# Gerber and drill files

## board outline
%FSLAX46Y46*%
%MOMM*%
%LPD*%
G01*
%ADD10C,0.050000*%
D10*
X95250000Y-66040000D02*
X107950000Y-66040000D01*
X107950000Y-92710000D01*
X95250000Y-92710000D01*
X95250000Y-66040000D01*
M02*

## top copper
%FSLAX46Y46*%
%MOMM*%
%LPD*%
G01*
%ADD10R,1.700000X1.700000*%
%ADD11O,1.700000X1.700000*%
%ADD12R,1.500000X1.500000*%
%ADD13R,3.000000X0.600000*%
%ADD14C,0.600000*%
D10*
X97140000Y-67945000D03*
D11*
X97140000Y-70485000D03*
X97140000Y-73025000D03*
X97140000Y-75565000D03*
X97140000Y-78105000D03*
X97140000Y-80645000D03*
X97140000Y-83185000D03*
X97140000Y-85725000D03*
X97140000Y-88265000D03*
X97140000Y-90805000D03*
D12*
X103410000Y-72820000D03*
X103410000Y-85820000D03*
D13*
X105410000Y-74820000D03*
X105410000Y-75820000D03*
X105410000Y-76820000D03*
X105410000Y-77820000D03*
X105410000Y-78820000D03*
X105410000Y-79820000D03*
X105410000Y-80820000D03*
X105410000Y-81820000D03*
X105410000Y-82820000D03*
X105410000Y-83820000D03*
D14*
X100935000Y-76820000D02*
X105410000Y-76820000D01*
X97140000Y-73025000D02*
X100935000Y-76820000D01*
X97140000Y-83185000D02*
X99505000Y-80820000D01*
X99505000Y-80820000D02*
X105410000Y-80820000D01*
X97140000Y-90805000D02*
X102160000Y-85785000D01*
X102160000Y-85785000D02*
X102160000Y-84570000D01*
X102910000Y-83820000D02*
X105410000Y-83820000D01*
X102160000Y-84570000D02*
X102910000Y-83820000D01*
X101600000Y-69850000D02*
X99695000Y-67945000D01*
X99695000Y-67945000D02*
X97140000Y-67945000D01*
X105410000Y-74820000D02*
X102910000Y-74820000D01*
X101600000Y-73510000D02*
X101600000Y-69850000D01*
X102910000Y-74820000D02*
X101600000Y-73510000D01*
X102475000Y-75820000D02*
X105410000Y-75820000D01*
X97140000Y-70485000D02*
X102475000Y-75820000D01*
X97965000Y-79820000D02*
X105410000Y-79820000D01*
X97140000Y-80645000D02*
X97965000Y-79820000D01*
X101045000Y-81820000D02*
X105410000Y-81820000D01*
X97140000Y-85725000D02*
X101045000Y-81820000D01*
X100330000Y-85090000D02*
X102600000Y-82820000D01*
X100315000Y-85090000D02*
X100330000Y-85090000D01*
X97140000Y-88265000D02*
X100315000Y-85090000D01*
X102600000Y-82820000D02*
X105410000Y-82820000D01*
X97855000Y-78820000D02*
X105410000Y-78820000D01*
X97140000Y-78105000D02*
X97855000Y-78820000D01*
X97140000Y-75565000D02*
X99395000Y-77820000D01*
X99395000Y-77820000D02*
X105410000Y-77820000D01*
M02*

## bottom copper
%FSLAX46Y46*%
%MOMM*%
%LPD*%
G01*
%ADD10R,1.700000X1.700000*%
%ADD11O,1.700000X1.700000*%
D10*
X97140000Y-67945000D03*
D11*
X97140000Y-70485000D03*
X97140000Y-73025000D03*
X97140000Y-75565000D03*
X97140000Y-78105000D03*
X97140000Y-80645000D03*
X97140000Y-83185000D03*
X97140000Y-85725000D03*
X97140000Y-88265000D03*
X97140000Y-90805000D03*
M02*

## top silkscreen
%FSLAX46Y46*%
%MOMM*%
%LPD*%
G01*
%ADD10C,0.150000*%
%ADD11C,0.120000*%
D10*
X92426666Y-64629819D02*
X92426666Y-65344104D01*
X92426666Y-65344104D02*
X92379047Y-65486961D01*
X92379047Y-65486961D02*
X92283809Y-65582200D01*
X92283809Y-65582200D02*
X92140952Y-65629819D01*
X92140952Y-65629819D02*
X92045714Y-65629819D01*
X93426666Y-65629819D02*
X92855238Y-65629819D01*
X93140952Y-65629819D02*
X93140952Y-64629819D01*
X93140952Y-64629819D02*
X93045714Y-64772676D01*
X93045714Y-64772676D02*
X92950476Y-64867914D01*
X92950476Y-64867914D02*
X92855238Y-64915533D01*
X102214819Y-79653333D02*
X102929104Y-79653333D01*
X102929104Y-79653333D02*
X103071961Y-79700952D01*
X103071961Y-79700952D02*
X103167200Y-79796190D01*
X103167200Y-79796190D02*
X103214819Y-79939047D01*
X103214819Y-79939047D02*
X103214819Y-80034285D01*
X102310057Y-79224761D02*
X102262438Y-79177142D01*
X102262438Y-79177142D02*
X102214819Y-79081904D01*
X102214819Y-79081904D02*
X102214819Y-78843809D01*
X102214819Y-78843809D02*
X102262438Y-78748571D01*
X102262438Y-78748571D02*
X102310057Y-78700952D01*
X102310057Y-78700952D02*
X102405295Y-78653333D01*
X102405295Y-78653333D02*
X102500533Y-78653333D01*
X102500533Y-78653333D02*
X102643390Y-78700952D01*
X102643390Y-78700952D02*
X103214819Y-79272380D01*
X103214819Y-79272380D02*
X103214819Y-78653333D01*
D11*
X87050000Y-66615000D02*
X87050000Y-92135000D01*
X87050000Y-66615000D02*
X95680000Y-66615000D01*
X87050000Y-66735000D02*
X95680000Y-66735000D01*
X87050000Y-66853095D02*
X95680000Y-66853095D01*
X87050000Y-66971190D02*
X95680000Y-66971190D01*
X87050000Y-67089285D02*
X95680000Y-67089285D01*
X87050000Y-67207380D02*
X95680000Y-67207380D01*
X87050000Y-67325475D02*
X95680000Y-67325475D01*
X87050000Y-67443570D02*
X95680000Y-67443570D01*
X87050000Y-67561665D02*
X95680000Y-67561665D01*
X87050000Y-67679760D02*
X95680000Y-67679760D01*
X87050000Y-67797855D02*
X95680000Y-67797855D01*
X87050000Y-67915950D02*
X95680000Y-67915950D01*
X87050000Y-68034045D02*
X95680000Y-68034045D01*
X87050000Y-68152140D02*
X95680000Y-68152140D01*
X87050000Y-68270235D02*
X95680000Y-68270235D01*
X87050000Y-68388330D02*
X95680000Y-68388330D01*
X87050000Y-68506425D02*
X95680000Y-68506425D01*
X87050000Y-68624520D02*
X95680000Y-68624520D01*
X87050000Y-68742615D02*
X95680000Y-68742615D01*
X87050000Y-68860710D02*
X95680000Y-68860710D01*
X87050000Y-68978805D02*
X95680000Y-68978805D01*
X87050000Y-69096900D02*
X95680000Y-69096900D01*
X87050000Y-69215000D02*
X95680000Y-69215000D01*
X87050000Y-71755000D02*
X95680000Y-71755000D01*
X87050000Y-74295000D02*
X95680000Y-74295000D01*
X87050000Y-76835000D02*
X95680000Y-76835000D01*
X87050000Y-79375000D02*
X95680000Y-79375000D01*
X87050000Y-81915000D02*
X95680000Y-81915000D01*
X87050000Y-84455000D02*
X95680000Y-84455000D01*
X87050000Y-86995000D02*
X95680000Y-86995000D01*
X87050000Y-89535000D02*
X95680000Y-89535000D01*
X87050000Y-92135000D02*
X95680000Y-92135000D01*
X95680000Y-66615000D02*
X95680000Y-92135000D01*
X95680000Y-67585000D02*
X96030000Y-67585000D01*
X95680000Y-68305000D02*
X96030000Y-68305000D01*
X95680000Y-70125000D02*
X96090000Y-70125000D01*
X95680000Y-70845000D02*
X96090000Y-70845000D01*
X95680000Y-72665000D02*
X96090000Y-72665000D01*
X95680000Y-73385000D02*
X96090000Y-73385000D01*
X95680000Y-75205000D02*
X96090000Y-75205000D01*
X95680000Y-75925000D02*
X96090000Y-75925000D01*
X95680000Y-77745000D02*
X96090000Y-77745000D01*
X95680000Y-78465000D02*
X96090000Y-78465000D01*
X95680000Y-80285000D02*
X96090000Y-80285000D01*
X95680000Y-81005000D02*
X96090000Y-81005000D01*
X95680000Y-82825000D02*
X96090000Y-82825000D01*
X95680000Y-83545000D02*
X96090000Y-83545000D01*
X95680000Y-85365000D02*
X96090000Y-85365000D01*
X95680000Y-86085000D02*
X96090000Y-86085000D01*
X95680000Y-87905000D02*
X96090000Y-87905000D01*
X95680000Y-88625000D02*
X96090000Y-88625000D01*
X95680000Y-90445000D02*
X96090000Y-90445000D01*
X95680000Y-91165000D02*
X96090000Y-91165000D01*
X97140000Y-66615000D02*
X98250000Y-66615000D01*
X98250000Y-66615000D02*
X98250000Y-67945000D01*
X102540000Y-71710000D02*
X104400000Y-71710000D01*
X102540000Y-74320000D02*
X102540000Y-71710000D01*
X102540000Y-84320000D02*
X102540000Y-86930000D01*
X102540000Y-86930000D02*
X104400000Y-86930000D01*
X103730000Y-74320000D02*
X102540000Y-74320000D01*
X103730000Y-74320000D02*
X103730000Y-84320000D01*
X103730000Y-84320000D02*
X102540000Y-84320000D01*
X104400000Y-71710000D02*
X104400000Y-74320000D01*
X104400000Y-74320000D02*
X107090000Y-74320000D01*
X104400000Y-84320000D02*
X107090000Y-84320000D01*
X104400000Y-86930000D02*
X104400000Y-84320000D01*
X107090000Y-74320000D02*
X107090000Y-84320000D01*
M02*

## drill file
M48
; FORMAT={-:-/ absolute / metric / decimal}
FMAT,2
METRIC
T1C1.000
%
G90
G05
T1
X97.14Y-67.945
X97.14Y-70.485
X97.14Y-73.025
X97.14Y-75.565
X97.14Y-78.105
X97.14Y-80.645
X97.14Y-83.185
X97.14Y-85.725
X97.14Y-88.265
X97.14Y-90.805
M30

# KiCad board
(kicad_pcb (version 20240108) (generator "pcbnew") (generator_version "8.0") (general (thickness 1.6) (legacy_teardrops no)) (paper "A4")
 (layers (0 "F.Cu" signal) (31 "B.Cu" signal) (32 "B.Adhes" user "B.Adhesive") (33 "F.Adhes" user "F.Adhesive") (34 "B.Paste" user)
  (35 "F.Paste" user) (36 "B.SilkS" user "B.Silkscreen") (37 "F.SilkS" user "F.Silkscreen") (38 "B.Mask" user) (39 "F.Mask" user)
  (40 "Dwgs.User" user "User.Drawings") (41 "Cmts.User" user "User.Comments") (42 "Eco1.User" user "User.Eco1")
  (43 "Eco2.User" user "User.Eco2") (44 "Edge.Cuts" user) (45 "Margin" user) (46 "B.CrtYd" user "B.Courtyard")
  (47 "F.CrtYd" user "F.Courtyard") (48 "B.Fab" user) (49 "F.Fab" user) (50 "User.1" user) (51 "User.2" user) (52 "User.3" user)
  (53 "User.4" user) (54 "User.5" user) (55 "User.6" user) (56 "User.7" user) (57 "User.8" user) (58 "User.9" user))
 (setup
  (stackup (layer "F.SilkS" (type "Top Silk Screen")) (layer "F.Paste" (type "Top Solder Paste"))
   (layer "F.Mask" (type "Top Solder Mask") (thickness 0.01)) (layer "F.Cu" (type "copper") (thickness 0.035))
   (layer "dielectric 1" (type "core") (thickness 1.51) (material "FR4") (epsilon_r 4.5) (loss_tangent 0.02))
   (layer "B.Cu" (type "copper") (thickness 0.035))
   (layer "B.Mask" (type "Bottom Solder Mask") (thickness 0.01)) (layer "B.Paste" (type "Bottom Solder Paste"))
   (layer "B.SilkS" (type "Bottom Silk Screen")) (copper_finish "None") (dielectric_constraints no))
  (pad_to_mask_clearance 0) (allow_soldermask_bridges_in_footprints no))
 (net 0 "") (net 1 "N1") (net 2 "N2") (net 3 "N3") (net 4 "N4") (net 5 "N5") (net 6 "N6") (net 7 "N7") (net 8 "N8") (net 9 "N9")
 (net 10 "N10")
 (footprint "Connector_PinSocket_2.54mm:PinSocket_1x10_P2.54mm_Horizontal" (layer "F.Cu") (at 97.14 67.945)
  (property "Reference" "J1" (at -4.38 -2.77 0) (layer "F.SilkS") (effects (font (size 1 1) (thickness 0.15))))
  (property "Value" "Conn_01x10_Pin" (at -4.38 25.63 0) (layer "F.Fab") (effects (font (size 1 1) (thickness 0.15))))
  (fp_line (start -10.09 -1.33) (end -10.09 24.19) (stroke (width 0.12) (type solid)) (layer "F.SilkS"))
  (fp_line (start -10.09 -1.33) (end -1.46 -1.33) (stroke (width 0.12) (type solid)) (layer "F.SilkS"))
  (fp_line (start -10.09 -1.21) (end -1.46 -1.21) (stroke (width 0.12) (type solid)) (layer "F.SilkS"))
  (fp_line (start -10.09 -1.091905) (end -1.46 -1.091905) (stroke (width 0.12) (type solid)) (layer "F.SilkS"))
  (fp_line (start -10.09 -0.97381) (end -1.46 -0.97381) (stroke (width 0.12) (type solid)) (layer "F.SilkS"))
  (fp_line (start -10.09 -0.855715) (end -1.46 -0.855715) (stroke (width 0.12) (type solid)) (layer "F.SilkS"))
  (fp_line (start -10.09 -0.73762) (end -1.46 -0.73762) (stroke (width 0.12) (type solid)) (layer "F.SilkS"))
  (fp_line (start -10.09 -0.619525) (end -1.46 -0.619525) (stroke (width 0.12) (type solid)) (layer "F.SilkS"))
  (fp_line (start -10.09 -0.50143) (end -1.46 -0.50143) (stroke (width 0.12) (type solid)) (layer "F.SilkS"))
  (fp_line (start -10.09 -0.383335) (end -1.46 -0.383335) (stroke (width 0.12) (type solid)) (layer "F.SilkS"))
  (fp_line (start -10.09 -0.26524) (end -1.46 -0.26524) (stroke (width 0.12) (type solid)) (layer "F.SilkS"))
  (fp_line (start -10.09 -0.147145) (end -1.46 -0.147145) (stroke (width 0.12) (type solid)) (layer "F.SilkS"))
  (fp_line (start -10.09 -0.02905) (end -1.46 -0.02905) (stroke (width 0.12) (type solid)) (layer "F.SilkS"))
  (fp_line (start -10.09 0.089045) (end -1.46 0.089045) (stroke (width 0.12) (type solid)) (layer "F.SilkS"))
  (fp_line (start -10.09 0.20714) (end -1.46 0.20714) (stroke (width 0.12) (type solid)) (layer "F.SilkS"))
  (fp_line (start -10.09 0.325235) (end -1.46 0.325235) (stroke (width 0.12) (type solid)) (layer "F.SilkS"))
  (fp_line (start -10.09 0.44333) (end -1.46 0.44333) (stroke (width 0.12) (type solid)) (layer "F.SilkS"))
  (fp_line (start -10.09 0.561425) (end -1.46 0.561425) (stroke (width 0.12) (type solid)) (layer "F.SilkS"))
  (fp_line (start -10.09 0.67952) (end -1.46 0.67952) (stroke (width 0.12) (type solid)) (layer "F.SilkS"))
  (fp_line (start -10.09 0.797615) (end -1.46 0.797615) (stroke (width 0.12) (type solid)) (layer "F.SilkS"))
  (fp_line (start -10.09 0.91571) (end -1.46 0.91571) (stroke (width 0.12) (type solid)) (layer "F.SilkS"))
  (fp_line (start -10.09 1.033805) (end -1.46 1.033805) (stroke (width 0.12) (type solid)) (layer "F.SilkS"))
  (fp_line (start -10.09 1.1519) (end -1.46 1.1519) (stroke (width 0.12) (type solid)) (layer "F.SilkS"))
  (fp_line (start -10.09 1.27) (end -1.46 1.27) (stroke (width 0.12) (type solid)) (layer "F.SilkS"))
  (fp_line (start -10.09 3.81) (end -1.46 3.81) (stroke (width 0.12) (type solid)) (layer "F.SilkS"))
  (fp_line (start -10.09 6.35) (end -1.46 6.35) (stroke (width 0.12) (type solid)) (layer "F.SilkS"))
  (fp_line (start -10.09 8.89) (end -1.46 8.89) (stroke (width 0.12) (type solid)) (layer "F.SilkS"))
  (fp_line (start -10.09 11.43) (end -1.46 11.43) (stroke (width 0.12) (type solid)) (layer "F.SilkS"))
  (fp_line (start -10.09 13.97) (end -1.46 13.97) (stroke (width 0.12) (type solid)) (layer "F.SilkS"))
  (fp_line (start -10.09 16.51) (end -1.46 16.51) (stroke (width 0.12) (type solid)) (layer "F.SilkS"))
  (fp_line (start -10.09 19.05) (end -1.46 19.05) (stroke (width 0.12) (type solid)) (layer "F.SilkS"))
  (fp_line (start -10.09 21.59) (end -1.46 21.59) (stroke (width 0.12) (type solid)) (layer "F.SilkS"))
  (fp_line (start -10.09 24.19) (end -1.46 24.19) (stroke (width 0.12) (type solid)) (layer "F.SilkS"))
  (fp_line (start -1.46 -1.33) (end -1.46 24.19) (stroke (width 0.12) (type solid)) (layer "F.SilkS"))
  (fp_line (start -1.46 -0.36) (end -1.11 -0.36) (stroke (width 0.12) (type solid)) (layer "F.SilkS"))
  (fp_line (start -1.46 0.36) (end -1.11 0.36) (stroke (width 0.12) (type solid)) (layer "F.SilkS"))
  (fp_line (start -1.46 2.18) (end -1.05 2.18) (stroke (width 0.12) (type solid)) (layer "F.SilkS"))
  (fp_line (start -1.46 2.9) (end -1.05 2.9) (stroke (width 0.12) (type solid)) (layer "F.SilkS"))
  (fp_line (start -1.46 4.72) (end -1.05 4.72) (stroke (width 0.12) (type solid)) (layer "F.SilkS"))
  (fp_line (start -1.46 5.44) (end -1.05 5.44) (stroke (width 0.12) (type solid)) (layer "F.SilkS"))
  (fp_line (start -1.46 7.26) (end -1.05 7.26) (stroke (width 0.12) (type solid)) (layer "F.SilkS"))
  (fp_line (start -1.46 7.98) (end -1.05 7.98) (stroke (width 0.12) (type solid)) (layer "F.SilkS"))
  (fp_line (start -1.46 9.8) (end -1.05 9.8) (stroke (width 0.12) (type solid)) (layer "F.SilkS"))
  (fp_line (start -1.46 10.52) (end -1.05 10.52) (stroke (width 0.12) (type solid)) (layer "F.SilkS"))
  (fp_line (start -1.46 12.34) (end -1.05 12.34) (stroke (width 0.12) (type solid)) (layer "F.SilkS"))
  (fp_line (start -1.46 13.06) (end -1.05 13.06) (stroke (width 0.12) (type solid)) (layer "F.SilkS"))
  (fp_line (start -1.46 14.88) (end -1.05 14.88) (stroke (width 0.12) (type solid)) (layer "F.SilkS"))
  (fp_line (start -1.46 15.6) (end -1.05 15.6) (stroke (width 0.12) (type solid)) (layer "F.SilkS"))
  (fp_line (start -1.46 17.42) (end -1.05 17.42) (stroke (width 0.12) (type solid)) (layer "F.SilkS"))
  (fp_line (start -1.46 18.14) (end -1.05 18.14) (stroke (width 0.12) (type solid)) (layer "F.SilkS"))
  (fp_line (start -1.46 19.96) (end -1.05 19.96) (stroke (width 0.12) (type solid)) (layer "F.SilkS"))
  (fp_line (start -1.46 20.68) (end -1.05 20.68) (stroke (width 0.12) (type solid)) (layer "F.SilkS"))
  (fp_line (start -1.46 22.5) (end -1.05 22.5) (stroke (width 0.12) (type solid)) (layer "F.SilkS"))
  (fp_line (start -1.46 23.22) (end -1.05 23.22) (stroke (width 0.12) (type solid)) (layer "F.SilkS"))
  (fp_line (start 0 -1.33) (end 1.11 -1.33) (stroke (width 0.12) (type solid)) (layer "F.SilkS"))
  (fp_line (start 1.11 -1.33) (end 1.11 0) (stroke (width 0.12) (type solid)) (layer "F.SilkS"))
  (pad "1" thru_hole rect (at 0 0) (size 1.7 1.7) (drill 1) (layers "*.Cu" "*.Mask") (remove_unused_layers no) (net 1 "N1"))
  (pad "2" thru_hole oval (at 0 2.54) (size 1.7 1.7) (drill 1) (layers "*.Cu" "*.Mask") (remove_unused_layers no) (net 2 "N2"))
  (pad "3" thru_hole oval (at 0 5.08) (size 1.7 1.7) (drill 1) (layers "*.Cu" "*.Mask") (remove_unused_layers no) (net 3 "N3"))
  (pad "4" thru_hole oval (at 0 7.62) (size 1.7 1.7) (drill 1) (layers "*.Cu" "*.Mask") (remove_unused_layers no) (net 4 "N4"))
  (pad "5" thru_hole oval (at 0 10.16) (size 1.7 1.7) (drill 1) (layers "*.Cu" "*.Mask") (remove_unused_layers no) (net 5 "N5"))
  (pad "6" thru_hole oval (at 0 12.7) (size 1.7 1.7) (drill 1) (layers "*.Cu" "*.Mask") (remove_unused_layers no) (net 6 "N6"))
  (pad "7" thru_hole oval (at 0 15.24) (size 1.7 1.7) (drill 1) (layers "*.Cu" "*.Mask") (remove_unused_layers no) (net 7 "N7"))
  (pad "8" thru_hole oval (at 0 17.78) (size 1.7 1.7) (drill 1) (layers "*.Cu" "*.Mask") (remove_unused_layers no) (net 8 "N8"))
  (pad "9" thru_hole oval (at 0 20.32) (size 1.7 1.7) (drill 1) (layers "*.Cu" "*.Mask") (remove_unused_layers no) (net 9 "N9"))
  (pad "10" thru_hole oval (at 0 22.86) (size 1.7 1.7) (drill 1) (layers "*.Cu" "*.Mask") (remove_unused_layers no) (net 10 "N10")))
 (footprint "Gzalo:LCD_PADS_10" (layer "F.Cu") (at 105.41 79.32 -90)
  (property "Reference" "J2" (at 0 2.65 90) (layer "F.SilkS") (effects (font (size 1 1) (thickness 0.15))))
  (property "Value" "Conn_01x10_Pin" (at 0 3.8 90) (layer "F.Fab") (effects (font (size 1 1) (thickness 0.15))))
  (fp_line (start -7.61 2.87) (end -7.61 1.01) (stroke (width 0.12) (type default)) (layer "F.SilkS"))
  (fp_line (start -5 2.87) (end -7.61 2.87) (stroke (width 0.12) (type default)) (layer "F.SilkS"))
  (fp_line (start 5 2.87) (end 7.61 2.87) (stroke (width 0.12) (type default)) (layer "F.SilkS"))
  (fp_line (start 7.61 2.87) (end 7.61 1.01) (stroke (width 0.12) (type default)) (layer "F.SilkS"))
  (fp_line (start -5 1.68) (end -5 2.87) (stroke (width 0.12) (type default)) (layer "F.SilkS"))
  (fp_line (start -5 1.68) (end 5 1.68) (stroke (width 0.12) (type default)) (layer "F.SilkS"))
  (fp_line (start 5 1.68) (end 5 2.87) (stroke (width 0.12) (type default)) (layer "F.SilkS"))
  (fp_line (start -7.61 1.01) (end -5 1.01) (stroke (width 0.12) (type default)) (layer "F.SilkS"))
  (fp_line (start -5 1.01) (end -5 -1.68) (stroke (width 0.12) (type default)) (layer "F.SilkS"))
  (fp_line (start 5 1.01) (end 5 -1.68) (stroke (width 0.12) (type default)) (layer "F.SilkS"))
  (fp_line (start 7.61 1.01) (end 5 1.01) (stroke (width 0.12) (type default)) (layer "F.SilkS"))
  (fp_line (start -5 -1.68) (end 5 -1.68) (stroke (width 0.12) (type default)) (layer "F.SilkS"))
  (pad "0" smd rect (at -6.5 2 270) (size 1.5 1.5) (layers "F.Cu" "F.Paste" "F.Mask") (thermal_bridge_angle 45))
  (pad "0" smd rect (at 6.5 2 270) (size 1.5 1.5) (layers "F.Cu" "F.Paste" "F.Mask") (thermal_bridge_angle 45))
  (pad "1" smd rect (at -4.5 0 270) (size 0.6 3) (layers "F.Cu" "F.Paste" "F.Mask") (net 1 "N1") (thermal_bridge_angle 45))
  (pad "2" smd rect (at -3.5 0 270) (size 0.6 3) (layers "F.Cu" "F.Paste" "F.Mask") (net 2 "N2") (thermal_bridge_angle 45))
  (pad "3" smd rect (at -2.5 0 270) (size 0.6 3) (layers "F.Cu" "F.Paste" "F.Mask") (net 3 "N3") (thermal_bridge_angle 45))
  (pad "4" smd rect (at -1.5 0 270) (size 0.6 3) (layers "F.Cu" "F.Paste" "F.Mask") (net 4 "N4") (thermal_bridge_angle 45))
  (pad "5" smd rect (at -0.5 0 270) (size 0.6 3) (layers "F.Cu" "F.Paste" "F.Mask") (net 5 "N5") (thermal_bridge_angle 45))
  (pad "6" smd rect (at 0.5 0 270) (size 0.6 3) (layers "F.Cu" "F.Paste" "F.Mask") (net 6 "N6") (thermal_bridge_angle 45))
  (pad "7" smd rect (at 1.5 0 270) (size 0.6 3) (layers "F.Cu" "F.Paste" "F.Mask") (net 7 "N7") (thermal_bridge_angle 45))
  (pad "8" smd rect (at 2.5 0 270) (size 0.6 3) (layers "F.Cu" "F.Paste" "F.Mask") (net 8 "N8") (thermal_bridge_angle 45))
  (pad "9" smd rect (at 3.5 0 270) (size 0.6 3) (layers "F.Cu" "F.Paste" "F.Mask") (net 9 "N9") (thermal_bridge_angle 45))
  (pad "10" smd rect (at 4.5 0 270) (size 0.6 3) (layers "F.Cu" "F.Paste" "F.Mask") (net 10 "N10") (thermal_bridge_angle 45)))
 (gr_rect (start 95.25 66.04) (end 107.95 92.71) (stroke (width 0.05) (type default)) (fill none) (layer "Edge.Cuts"))
 (segment (start 100.935 76.82) (end 105.41 76.82) (width 0.6) (layer "F.Cu") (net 3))
 (segment (start 97.14 73.025) (end 100.935 76.82) (width 0.6) (layer "F.Cu") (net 3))
 (segment (start 97.14 83.185) (end 99.505 80.82) (width 0.6) (layer "F.Cu") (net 7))
 (segment (start 99.505 80.82) (end 105.41 80.82) (width 0.6) (layer "F.Cu") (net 7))
 (segment (start 97.14 90.805) (end 102.16 85.785) (width 0.6) (layer "F.Cu") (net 10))
 (segment (start 102.16 85.785) (end 102.16 84.57) (width 0.6) (layer "F.Cu") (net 10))
 (segment (start 102.91 83.82) (end 105.41 83.82) (width 0.6) (layer "F.Cu") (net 10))
 (segment (start 102.16 84.57) (end 102.91 83.82) (width 0.6) (layer "F.Cu") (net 10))
 (segment (start 101.6 69.85) (end 99.695 67.945) (width 0.6) (layer "F.Cu") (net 1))
 (segment (start 99.695 67.945) (end 97.14 67.945) (width 0.6) (layer "F.Cu") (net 1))
 (segment (start 105.41 74.82) (end 102.91 74.82) (width 0.6) (layer "F.Cu") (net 1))
 (segment (start 101.6 73.51) (end 101.6 69.85) (width 0.6) (layer "F.Cu") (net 1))
 (segment (start 102.91 74.82) (end 101.6 73.51) (width 0.6) (layer "F.Cu") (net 1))
 (segment (start 102.475 75.82) (end 105.41 75.82) (width 0.6) (layer "F.Cu") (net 2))
 (segment (start 97.14 70.485) (end 102.475 75.82) (width 0.6) (layer "F.Cu") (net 2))
 (segment (start 97.965 79.82) (end 105.41 79.82) (width 0.6) (layer "F.Cu") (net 6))
 (segment (start 97.14 80.645) (end 97.965 79.82) (width 0.6) (layer "F.Cu") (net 6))
 (segment (start 101.045 81.82) (end 105.41 81.82) (width 0.6) (layer "F.Cu") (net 8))
 (segment (start 97.14 85.725) (end 101.045 81.82) (width 0.6) (layer "F.Cu") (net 8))
 (segment (start 100.33 85.09) (end 102.6 82.82) (width 0.6) (layer "F.Cu") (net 9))
 (segment (start 100.315 85.09) (end 100.33 85.09) (width 0.6) (layer "F.Cu") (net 9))
 (segment (start 97.14 88.265) (end 100.315 85.09) (width 0.6) (layer "F.Cu") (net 9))
 (segment (start 102.6 82.82) (end 105.41 82.82) (width 0.6) (layer "F.Cu") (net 9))
 (segment (start 97.855 78.82) (end 105.41 78.82) (width 0.6) (layer "F.Cu") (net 5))
 (segment (start 97.14 78.105) (end 97.855 78.82) (width 0.6) (layer "F.Cu") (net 5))
 (segment (start 97.14 75.565) (end 99.395 77.82) (width 0.6) (layer "F.Cu") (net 4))
 (segment (start 99.395 77.82) (end 105.41 77.82) (width 0.6) (layer "F.Cu") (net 4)))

